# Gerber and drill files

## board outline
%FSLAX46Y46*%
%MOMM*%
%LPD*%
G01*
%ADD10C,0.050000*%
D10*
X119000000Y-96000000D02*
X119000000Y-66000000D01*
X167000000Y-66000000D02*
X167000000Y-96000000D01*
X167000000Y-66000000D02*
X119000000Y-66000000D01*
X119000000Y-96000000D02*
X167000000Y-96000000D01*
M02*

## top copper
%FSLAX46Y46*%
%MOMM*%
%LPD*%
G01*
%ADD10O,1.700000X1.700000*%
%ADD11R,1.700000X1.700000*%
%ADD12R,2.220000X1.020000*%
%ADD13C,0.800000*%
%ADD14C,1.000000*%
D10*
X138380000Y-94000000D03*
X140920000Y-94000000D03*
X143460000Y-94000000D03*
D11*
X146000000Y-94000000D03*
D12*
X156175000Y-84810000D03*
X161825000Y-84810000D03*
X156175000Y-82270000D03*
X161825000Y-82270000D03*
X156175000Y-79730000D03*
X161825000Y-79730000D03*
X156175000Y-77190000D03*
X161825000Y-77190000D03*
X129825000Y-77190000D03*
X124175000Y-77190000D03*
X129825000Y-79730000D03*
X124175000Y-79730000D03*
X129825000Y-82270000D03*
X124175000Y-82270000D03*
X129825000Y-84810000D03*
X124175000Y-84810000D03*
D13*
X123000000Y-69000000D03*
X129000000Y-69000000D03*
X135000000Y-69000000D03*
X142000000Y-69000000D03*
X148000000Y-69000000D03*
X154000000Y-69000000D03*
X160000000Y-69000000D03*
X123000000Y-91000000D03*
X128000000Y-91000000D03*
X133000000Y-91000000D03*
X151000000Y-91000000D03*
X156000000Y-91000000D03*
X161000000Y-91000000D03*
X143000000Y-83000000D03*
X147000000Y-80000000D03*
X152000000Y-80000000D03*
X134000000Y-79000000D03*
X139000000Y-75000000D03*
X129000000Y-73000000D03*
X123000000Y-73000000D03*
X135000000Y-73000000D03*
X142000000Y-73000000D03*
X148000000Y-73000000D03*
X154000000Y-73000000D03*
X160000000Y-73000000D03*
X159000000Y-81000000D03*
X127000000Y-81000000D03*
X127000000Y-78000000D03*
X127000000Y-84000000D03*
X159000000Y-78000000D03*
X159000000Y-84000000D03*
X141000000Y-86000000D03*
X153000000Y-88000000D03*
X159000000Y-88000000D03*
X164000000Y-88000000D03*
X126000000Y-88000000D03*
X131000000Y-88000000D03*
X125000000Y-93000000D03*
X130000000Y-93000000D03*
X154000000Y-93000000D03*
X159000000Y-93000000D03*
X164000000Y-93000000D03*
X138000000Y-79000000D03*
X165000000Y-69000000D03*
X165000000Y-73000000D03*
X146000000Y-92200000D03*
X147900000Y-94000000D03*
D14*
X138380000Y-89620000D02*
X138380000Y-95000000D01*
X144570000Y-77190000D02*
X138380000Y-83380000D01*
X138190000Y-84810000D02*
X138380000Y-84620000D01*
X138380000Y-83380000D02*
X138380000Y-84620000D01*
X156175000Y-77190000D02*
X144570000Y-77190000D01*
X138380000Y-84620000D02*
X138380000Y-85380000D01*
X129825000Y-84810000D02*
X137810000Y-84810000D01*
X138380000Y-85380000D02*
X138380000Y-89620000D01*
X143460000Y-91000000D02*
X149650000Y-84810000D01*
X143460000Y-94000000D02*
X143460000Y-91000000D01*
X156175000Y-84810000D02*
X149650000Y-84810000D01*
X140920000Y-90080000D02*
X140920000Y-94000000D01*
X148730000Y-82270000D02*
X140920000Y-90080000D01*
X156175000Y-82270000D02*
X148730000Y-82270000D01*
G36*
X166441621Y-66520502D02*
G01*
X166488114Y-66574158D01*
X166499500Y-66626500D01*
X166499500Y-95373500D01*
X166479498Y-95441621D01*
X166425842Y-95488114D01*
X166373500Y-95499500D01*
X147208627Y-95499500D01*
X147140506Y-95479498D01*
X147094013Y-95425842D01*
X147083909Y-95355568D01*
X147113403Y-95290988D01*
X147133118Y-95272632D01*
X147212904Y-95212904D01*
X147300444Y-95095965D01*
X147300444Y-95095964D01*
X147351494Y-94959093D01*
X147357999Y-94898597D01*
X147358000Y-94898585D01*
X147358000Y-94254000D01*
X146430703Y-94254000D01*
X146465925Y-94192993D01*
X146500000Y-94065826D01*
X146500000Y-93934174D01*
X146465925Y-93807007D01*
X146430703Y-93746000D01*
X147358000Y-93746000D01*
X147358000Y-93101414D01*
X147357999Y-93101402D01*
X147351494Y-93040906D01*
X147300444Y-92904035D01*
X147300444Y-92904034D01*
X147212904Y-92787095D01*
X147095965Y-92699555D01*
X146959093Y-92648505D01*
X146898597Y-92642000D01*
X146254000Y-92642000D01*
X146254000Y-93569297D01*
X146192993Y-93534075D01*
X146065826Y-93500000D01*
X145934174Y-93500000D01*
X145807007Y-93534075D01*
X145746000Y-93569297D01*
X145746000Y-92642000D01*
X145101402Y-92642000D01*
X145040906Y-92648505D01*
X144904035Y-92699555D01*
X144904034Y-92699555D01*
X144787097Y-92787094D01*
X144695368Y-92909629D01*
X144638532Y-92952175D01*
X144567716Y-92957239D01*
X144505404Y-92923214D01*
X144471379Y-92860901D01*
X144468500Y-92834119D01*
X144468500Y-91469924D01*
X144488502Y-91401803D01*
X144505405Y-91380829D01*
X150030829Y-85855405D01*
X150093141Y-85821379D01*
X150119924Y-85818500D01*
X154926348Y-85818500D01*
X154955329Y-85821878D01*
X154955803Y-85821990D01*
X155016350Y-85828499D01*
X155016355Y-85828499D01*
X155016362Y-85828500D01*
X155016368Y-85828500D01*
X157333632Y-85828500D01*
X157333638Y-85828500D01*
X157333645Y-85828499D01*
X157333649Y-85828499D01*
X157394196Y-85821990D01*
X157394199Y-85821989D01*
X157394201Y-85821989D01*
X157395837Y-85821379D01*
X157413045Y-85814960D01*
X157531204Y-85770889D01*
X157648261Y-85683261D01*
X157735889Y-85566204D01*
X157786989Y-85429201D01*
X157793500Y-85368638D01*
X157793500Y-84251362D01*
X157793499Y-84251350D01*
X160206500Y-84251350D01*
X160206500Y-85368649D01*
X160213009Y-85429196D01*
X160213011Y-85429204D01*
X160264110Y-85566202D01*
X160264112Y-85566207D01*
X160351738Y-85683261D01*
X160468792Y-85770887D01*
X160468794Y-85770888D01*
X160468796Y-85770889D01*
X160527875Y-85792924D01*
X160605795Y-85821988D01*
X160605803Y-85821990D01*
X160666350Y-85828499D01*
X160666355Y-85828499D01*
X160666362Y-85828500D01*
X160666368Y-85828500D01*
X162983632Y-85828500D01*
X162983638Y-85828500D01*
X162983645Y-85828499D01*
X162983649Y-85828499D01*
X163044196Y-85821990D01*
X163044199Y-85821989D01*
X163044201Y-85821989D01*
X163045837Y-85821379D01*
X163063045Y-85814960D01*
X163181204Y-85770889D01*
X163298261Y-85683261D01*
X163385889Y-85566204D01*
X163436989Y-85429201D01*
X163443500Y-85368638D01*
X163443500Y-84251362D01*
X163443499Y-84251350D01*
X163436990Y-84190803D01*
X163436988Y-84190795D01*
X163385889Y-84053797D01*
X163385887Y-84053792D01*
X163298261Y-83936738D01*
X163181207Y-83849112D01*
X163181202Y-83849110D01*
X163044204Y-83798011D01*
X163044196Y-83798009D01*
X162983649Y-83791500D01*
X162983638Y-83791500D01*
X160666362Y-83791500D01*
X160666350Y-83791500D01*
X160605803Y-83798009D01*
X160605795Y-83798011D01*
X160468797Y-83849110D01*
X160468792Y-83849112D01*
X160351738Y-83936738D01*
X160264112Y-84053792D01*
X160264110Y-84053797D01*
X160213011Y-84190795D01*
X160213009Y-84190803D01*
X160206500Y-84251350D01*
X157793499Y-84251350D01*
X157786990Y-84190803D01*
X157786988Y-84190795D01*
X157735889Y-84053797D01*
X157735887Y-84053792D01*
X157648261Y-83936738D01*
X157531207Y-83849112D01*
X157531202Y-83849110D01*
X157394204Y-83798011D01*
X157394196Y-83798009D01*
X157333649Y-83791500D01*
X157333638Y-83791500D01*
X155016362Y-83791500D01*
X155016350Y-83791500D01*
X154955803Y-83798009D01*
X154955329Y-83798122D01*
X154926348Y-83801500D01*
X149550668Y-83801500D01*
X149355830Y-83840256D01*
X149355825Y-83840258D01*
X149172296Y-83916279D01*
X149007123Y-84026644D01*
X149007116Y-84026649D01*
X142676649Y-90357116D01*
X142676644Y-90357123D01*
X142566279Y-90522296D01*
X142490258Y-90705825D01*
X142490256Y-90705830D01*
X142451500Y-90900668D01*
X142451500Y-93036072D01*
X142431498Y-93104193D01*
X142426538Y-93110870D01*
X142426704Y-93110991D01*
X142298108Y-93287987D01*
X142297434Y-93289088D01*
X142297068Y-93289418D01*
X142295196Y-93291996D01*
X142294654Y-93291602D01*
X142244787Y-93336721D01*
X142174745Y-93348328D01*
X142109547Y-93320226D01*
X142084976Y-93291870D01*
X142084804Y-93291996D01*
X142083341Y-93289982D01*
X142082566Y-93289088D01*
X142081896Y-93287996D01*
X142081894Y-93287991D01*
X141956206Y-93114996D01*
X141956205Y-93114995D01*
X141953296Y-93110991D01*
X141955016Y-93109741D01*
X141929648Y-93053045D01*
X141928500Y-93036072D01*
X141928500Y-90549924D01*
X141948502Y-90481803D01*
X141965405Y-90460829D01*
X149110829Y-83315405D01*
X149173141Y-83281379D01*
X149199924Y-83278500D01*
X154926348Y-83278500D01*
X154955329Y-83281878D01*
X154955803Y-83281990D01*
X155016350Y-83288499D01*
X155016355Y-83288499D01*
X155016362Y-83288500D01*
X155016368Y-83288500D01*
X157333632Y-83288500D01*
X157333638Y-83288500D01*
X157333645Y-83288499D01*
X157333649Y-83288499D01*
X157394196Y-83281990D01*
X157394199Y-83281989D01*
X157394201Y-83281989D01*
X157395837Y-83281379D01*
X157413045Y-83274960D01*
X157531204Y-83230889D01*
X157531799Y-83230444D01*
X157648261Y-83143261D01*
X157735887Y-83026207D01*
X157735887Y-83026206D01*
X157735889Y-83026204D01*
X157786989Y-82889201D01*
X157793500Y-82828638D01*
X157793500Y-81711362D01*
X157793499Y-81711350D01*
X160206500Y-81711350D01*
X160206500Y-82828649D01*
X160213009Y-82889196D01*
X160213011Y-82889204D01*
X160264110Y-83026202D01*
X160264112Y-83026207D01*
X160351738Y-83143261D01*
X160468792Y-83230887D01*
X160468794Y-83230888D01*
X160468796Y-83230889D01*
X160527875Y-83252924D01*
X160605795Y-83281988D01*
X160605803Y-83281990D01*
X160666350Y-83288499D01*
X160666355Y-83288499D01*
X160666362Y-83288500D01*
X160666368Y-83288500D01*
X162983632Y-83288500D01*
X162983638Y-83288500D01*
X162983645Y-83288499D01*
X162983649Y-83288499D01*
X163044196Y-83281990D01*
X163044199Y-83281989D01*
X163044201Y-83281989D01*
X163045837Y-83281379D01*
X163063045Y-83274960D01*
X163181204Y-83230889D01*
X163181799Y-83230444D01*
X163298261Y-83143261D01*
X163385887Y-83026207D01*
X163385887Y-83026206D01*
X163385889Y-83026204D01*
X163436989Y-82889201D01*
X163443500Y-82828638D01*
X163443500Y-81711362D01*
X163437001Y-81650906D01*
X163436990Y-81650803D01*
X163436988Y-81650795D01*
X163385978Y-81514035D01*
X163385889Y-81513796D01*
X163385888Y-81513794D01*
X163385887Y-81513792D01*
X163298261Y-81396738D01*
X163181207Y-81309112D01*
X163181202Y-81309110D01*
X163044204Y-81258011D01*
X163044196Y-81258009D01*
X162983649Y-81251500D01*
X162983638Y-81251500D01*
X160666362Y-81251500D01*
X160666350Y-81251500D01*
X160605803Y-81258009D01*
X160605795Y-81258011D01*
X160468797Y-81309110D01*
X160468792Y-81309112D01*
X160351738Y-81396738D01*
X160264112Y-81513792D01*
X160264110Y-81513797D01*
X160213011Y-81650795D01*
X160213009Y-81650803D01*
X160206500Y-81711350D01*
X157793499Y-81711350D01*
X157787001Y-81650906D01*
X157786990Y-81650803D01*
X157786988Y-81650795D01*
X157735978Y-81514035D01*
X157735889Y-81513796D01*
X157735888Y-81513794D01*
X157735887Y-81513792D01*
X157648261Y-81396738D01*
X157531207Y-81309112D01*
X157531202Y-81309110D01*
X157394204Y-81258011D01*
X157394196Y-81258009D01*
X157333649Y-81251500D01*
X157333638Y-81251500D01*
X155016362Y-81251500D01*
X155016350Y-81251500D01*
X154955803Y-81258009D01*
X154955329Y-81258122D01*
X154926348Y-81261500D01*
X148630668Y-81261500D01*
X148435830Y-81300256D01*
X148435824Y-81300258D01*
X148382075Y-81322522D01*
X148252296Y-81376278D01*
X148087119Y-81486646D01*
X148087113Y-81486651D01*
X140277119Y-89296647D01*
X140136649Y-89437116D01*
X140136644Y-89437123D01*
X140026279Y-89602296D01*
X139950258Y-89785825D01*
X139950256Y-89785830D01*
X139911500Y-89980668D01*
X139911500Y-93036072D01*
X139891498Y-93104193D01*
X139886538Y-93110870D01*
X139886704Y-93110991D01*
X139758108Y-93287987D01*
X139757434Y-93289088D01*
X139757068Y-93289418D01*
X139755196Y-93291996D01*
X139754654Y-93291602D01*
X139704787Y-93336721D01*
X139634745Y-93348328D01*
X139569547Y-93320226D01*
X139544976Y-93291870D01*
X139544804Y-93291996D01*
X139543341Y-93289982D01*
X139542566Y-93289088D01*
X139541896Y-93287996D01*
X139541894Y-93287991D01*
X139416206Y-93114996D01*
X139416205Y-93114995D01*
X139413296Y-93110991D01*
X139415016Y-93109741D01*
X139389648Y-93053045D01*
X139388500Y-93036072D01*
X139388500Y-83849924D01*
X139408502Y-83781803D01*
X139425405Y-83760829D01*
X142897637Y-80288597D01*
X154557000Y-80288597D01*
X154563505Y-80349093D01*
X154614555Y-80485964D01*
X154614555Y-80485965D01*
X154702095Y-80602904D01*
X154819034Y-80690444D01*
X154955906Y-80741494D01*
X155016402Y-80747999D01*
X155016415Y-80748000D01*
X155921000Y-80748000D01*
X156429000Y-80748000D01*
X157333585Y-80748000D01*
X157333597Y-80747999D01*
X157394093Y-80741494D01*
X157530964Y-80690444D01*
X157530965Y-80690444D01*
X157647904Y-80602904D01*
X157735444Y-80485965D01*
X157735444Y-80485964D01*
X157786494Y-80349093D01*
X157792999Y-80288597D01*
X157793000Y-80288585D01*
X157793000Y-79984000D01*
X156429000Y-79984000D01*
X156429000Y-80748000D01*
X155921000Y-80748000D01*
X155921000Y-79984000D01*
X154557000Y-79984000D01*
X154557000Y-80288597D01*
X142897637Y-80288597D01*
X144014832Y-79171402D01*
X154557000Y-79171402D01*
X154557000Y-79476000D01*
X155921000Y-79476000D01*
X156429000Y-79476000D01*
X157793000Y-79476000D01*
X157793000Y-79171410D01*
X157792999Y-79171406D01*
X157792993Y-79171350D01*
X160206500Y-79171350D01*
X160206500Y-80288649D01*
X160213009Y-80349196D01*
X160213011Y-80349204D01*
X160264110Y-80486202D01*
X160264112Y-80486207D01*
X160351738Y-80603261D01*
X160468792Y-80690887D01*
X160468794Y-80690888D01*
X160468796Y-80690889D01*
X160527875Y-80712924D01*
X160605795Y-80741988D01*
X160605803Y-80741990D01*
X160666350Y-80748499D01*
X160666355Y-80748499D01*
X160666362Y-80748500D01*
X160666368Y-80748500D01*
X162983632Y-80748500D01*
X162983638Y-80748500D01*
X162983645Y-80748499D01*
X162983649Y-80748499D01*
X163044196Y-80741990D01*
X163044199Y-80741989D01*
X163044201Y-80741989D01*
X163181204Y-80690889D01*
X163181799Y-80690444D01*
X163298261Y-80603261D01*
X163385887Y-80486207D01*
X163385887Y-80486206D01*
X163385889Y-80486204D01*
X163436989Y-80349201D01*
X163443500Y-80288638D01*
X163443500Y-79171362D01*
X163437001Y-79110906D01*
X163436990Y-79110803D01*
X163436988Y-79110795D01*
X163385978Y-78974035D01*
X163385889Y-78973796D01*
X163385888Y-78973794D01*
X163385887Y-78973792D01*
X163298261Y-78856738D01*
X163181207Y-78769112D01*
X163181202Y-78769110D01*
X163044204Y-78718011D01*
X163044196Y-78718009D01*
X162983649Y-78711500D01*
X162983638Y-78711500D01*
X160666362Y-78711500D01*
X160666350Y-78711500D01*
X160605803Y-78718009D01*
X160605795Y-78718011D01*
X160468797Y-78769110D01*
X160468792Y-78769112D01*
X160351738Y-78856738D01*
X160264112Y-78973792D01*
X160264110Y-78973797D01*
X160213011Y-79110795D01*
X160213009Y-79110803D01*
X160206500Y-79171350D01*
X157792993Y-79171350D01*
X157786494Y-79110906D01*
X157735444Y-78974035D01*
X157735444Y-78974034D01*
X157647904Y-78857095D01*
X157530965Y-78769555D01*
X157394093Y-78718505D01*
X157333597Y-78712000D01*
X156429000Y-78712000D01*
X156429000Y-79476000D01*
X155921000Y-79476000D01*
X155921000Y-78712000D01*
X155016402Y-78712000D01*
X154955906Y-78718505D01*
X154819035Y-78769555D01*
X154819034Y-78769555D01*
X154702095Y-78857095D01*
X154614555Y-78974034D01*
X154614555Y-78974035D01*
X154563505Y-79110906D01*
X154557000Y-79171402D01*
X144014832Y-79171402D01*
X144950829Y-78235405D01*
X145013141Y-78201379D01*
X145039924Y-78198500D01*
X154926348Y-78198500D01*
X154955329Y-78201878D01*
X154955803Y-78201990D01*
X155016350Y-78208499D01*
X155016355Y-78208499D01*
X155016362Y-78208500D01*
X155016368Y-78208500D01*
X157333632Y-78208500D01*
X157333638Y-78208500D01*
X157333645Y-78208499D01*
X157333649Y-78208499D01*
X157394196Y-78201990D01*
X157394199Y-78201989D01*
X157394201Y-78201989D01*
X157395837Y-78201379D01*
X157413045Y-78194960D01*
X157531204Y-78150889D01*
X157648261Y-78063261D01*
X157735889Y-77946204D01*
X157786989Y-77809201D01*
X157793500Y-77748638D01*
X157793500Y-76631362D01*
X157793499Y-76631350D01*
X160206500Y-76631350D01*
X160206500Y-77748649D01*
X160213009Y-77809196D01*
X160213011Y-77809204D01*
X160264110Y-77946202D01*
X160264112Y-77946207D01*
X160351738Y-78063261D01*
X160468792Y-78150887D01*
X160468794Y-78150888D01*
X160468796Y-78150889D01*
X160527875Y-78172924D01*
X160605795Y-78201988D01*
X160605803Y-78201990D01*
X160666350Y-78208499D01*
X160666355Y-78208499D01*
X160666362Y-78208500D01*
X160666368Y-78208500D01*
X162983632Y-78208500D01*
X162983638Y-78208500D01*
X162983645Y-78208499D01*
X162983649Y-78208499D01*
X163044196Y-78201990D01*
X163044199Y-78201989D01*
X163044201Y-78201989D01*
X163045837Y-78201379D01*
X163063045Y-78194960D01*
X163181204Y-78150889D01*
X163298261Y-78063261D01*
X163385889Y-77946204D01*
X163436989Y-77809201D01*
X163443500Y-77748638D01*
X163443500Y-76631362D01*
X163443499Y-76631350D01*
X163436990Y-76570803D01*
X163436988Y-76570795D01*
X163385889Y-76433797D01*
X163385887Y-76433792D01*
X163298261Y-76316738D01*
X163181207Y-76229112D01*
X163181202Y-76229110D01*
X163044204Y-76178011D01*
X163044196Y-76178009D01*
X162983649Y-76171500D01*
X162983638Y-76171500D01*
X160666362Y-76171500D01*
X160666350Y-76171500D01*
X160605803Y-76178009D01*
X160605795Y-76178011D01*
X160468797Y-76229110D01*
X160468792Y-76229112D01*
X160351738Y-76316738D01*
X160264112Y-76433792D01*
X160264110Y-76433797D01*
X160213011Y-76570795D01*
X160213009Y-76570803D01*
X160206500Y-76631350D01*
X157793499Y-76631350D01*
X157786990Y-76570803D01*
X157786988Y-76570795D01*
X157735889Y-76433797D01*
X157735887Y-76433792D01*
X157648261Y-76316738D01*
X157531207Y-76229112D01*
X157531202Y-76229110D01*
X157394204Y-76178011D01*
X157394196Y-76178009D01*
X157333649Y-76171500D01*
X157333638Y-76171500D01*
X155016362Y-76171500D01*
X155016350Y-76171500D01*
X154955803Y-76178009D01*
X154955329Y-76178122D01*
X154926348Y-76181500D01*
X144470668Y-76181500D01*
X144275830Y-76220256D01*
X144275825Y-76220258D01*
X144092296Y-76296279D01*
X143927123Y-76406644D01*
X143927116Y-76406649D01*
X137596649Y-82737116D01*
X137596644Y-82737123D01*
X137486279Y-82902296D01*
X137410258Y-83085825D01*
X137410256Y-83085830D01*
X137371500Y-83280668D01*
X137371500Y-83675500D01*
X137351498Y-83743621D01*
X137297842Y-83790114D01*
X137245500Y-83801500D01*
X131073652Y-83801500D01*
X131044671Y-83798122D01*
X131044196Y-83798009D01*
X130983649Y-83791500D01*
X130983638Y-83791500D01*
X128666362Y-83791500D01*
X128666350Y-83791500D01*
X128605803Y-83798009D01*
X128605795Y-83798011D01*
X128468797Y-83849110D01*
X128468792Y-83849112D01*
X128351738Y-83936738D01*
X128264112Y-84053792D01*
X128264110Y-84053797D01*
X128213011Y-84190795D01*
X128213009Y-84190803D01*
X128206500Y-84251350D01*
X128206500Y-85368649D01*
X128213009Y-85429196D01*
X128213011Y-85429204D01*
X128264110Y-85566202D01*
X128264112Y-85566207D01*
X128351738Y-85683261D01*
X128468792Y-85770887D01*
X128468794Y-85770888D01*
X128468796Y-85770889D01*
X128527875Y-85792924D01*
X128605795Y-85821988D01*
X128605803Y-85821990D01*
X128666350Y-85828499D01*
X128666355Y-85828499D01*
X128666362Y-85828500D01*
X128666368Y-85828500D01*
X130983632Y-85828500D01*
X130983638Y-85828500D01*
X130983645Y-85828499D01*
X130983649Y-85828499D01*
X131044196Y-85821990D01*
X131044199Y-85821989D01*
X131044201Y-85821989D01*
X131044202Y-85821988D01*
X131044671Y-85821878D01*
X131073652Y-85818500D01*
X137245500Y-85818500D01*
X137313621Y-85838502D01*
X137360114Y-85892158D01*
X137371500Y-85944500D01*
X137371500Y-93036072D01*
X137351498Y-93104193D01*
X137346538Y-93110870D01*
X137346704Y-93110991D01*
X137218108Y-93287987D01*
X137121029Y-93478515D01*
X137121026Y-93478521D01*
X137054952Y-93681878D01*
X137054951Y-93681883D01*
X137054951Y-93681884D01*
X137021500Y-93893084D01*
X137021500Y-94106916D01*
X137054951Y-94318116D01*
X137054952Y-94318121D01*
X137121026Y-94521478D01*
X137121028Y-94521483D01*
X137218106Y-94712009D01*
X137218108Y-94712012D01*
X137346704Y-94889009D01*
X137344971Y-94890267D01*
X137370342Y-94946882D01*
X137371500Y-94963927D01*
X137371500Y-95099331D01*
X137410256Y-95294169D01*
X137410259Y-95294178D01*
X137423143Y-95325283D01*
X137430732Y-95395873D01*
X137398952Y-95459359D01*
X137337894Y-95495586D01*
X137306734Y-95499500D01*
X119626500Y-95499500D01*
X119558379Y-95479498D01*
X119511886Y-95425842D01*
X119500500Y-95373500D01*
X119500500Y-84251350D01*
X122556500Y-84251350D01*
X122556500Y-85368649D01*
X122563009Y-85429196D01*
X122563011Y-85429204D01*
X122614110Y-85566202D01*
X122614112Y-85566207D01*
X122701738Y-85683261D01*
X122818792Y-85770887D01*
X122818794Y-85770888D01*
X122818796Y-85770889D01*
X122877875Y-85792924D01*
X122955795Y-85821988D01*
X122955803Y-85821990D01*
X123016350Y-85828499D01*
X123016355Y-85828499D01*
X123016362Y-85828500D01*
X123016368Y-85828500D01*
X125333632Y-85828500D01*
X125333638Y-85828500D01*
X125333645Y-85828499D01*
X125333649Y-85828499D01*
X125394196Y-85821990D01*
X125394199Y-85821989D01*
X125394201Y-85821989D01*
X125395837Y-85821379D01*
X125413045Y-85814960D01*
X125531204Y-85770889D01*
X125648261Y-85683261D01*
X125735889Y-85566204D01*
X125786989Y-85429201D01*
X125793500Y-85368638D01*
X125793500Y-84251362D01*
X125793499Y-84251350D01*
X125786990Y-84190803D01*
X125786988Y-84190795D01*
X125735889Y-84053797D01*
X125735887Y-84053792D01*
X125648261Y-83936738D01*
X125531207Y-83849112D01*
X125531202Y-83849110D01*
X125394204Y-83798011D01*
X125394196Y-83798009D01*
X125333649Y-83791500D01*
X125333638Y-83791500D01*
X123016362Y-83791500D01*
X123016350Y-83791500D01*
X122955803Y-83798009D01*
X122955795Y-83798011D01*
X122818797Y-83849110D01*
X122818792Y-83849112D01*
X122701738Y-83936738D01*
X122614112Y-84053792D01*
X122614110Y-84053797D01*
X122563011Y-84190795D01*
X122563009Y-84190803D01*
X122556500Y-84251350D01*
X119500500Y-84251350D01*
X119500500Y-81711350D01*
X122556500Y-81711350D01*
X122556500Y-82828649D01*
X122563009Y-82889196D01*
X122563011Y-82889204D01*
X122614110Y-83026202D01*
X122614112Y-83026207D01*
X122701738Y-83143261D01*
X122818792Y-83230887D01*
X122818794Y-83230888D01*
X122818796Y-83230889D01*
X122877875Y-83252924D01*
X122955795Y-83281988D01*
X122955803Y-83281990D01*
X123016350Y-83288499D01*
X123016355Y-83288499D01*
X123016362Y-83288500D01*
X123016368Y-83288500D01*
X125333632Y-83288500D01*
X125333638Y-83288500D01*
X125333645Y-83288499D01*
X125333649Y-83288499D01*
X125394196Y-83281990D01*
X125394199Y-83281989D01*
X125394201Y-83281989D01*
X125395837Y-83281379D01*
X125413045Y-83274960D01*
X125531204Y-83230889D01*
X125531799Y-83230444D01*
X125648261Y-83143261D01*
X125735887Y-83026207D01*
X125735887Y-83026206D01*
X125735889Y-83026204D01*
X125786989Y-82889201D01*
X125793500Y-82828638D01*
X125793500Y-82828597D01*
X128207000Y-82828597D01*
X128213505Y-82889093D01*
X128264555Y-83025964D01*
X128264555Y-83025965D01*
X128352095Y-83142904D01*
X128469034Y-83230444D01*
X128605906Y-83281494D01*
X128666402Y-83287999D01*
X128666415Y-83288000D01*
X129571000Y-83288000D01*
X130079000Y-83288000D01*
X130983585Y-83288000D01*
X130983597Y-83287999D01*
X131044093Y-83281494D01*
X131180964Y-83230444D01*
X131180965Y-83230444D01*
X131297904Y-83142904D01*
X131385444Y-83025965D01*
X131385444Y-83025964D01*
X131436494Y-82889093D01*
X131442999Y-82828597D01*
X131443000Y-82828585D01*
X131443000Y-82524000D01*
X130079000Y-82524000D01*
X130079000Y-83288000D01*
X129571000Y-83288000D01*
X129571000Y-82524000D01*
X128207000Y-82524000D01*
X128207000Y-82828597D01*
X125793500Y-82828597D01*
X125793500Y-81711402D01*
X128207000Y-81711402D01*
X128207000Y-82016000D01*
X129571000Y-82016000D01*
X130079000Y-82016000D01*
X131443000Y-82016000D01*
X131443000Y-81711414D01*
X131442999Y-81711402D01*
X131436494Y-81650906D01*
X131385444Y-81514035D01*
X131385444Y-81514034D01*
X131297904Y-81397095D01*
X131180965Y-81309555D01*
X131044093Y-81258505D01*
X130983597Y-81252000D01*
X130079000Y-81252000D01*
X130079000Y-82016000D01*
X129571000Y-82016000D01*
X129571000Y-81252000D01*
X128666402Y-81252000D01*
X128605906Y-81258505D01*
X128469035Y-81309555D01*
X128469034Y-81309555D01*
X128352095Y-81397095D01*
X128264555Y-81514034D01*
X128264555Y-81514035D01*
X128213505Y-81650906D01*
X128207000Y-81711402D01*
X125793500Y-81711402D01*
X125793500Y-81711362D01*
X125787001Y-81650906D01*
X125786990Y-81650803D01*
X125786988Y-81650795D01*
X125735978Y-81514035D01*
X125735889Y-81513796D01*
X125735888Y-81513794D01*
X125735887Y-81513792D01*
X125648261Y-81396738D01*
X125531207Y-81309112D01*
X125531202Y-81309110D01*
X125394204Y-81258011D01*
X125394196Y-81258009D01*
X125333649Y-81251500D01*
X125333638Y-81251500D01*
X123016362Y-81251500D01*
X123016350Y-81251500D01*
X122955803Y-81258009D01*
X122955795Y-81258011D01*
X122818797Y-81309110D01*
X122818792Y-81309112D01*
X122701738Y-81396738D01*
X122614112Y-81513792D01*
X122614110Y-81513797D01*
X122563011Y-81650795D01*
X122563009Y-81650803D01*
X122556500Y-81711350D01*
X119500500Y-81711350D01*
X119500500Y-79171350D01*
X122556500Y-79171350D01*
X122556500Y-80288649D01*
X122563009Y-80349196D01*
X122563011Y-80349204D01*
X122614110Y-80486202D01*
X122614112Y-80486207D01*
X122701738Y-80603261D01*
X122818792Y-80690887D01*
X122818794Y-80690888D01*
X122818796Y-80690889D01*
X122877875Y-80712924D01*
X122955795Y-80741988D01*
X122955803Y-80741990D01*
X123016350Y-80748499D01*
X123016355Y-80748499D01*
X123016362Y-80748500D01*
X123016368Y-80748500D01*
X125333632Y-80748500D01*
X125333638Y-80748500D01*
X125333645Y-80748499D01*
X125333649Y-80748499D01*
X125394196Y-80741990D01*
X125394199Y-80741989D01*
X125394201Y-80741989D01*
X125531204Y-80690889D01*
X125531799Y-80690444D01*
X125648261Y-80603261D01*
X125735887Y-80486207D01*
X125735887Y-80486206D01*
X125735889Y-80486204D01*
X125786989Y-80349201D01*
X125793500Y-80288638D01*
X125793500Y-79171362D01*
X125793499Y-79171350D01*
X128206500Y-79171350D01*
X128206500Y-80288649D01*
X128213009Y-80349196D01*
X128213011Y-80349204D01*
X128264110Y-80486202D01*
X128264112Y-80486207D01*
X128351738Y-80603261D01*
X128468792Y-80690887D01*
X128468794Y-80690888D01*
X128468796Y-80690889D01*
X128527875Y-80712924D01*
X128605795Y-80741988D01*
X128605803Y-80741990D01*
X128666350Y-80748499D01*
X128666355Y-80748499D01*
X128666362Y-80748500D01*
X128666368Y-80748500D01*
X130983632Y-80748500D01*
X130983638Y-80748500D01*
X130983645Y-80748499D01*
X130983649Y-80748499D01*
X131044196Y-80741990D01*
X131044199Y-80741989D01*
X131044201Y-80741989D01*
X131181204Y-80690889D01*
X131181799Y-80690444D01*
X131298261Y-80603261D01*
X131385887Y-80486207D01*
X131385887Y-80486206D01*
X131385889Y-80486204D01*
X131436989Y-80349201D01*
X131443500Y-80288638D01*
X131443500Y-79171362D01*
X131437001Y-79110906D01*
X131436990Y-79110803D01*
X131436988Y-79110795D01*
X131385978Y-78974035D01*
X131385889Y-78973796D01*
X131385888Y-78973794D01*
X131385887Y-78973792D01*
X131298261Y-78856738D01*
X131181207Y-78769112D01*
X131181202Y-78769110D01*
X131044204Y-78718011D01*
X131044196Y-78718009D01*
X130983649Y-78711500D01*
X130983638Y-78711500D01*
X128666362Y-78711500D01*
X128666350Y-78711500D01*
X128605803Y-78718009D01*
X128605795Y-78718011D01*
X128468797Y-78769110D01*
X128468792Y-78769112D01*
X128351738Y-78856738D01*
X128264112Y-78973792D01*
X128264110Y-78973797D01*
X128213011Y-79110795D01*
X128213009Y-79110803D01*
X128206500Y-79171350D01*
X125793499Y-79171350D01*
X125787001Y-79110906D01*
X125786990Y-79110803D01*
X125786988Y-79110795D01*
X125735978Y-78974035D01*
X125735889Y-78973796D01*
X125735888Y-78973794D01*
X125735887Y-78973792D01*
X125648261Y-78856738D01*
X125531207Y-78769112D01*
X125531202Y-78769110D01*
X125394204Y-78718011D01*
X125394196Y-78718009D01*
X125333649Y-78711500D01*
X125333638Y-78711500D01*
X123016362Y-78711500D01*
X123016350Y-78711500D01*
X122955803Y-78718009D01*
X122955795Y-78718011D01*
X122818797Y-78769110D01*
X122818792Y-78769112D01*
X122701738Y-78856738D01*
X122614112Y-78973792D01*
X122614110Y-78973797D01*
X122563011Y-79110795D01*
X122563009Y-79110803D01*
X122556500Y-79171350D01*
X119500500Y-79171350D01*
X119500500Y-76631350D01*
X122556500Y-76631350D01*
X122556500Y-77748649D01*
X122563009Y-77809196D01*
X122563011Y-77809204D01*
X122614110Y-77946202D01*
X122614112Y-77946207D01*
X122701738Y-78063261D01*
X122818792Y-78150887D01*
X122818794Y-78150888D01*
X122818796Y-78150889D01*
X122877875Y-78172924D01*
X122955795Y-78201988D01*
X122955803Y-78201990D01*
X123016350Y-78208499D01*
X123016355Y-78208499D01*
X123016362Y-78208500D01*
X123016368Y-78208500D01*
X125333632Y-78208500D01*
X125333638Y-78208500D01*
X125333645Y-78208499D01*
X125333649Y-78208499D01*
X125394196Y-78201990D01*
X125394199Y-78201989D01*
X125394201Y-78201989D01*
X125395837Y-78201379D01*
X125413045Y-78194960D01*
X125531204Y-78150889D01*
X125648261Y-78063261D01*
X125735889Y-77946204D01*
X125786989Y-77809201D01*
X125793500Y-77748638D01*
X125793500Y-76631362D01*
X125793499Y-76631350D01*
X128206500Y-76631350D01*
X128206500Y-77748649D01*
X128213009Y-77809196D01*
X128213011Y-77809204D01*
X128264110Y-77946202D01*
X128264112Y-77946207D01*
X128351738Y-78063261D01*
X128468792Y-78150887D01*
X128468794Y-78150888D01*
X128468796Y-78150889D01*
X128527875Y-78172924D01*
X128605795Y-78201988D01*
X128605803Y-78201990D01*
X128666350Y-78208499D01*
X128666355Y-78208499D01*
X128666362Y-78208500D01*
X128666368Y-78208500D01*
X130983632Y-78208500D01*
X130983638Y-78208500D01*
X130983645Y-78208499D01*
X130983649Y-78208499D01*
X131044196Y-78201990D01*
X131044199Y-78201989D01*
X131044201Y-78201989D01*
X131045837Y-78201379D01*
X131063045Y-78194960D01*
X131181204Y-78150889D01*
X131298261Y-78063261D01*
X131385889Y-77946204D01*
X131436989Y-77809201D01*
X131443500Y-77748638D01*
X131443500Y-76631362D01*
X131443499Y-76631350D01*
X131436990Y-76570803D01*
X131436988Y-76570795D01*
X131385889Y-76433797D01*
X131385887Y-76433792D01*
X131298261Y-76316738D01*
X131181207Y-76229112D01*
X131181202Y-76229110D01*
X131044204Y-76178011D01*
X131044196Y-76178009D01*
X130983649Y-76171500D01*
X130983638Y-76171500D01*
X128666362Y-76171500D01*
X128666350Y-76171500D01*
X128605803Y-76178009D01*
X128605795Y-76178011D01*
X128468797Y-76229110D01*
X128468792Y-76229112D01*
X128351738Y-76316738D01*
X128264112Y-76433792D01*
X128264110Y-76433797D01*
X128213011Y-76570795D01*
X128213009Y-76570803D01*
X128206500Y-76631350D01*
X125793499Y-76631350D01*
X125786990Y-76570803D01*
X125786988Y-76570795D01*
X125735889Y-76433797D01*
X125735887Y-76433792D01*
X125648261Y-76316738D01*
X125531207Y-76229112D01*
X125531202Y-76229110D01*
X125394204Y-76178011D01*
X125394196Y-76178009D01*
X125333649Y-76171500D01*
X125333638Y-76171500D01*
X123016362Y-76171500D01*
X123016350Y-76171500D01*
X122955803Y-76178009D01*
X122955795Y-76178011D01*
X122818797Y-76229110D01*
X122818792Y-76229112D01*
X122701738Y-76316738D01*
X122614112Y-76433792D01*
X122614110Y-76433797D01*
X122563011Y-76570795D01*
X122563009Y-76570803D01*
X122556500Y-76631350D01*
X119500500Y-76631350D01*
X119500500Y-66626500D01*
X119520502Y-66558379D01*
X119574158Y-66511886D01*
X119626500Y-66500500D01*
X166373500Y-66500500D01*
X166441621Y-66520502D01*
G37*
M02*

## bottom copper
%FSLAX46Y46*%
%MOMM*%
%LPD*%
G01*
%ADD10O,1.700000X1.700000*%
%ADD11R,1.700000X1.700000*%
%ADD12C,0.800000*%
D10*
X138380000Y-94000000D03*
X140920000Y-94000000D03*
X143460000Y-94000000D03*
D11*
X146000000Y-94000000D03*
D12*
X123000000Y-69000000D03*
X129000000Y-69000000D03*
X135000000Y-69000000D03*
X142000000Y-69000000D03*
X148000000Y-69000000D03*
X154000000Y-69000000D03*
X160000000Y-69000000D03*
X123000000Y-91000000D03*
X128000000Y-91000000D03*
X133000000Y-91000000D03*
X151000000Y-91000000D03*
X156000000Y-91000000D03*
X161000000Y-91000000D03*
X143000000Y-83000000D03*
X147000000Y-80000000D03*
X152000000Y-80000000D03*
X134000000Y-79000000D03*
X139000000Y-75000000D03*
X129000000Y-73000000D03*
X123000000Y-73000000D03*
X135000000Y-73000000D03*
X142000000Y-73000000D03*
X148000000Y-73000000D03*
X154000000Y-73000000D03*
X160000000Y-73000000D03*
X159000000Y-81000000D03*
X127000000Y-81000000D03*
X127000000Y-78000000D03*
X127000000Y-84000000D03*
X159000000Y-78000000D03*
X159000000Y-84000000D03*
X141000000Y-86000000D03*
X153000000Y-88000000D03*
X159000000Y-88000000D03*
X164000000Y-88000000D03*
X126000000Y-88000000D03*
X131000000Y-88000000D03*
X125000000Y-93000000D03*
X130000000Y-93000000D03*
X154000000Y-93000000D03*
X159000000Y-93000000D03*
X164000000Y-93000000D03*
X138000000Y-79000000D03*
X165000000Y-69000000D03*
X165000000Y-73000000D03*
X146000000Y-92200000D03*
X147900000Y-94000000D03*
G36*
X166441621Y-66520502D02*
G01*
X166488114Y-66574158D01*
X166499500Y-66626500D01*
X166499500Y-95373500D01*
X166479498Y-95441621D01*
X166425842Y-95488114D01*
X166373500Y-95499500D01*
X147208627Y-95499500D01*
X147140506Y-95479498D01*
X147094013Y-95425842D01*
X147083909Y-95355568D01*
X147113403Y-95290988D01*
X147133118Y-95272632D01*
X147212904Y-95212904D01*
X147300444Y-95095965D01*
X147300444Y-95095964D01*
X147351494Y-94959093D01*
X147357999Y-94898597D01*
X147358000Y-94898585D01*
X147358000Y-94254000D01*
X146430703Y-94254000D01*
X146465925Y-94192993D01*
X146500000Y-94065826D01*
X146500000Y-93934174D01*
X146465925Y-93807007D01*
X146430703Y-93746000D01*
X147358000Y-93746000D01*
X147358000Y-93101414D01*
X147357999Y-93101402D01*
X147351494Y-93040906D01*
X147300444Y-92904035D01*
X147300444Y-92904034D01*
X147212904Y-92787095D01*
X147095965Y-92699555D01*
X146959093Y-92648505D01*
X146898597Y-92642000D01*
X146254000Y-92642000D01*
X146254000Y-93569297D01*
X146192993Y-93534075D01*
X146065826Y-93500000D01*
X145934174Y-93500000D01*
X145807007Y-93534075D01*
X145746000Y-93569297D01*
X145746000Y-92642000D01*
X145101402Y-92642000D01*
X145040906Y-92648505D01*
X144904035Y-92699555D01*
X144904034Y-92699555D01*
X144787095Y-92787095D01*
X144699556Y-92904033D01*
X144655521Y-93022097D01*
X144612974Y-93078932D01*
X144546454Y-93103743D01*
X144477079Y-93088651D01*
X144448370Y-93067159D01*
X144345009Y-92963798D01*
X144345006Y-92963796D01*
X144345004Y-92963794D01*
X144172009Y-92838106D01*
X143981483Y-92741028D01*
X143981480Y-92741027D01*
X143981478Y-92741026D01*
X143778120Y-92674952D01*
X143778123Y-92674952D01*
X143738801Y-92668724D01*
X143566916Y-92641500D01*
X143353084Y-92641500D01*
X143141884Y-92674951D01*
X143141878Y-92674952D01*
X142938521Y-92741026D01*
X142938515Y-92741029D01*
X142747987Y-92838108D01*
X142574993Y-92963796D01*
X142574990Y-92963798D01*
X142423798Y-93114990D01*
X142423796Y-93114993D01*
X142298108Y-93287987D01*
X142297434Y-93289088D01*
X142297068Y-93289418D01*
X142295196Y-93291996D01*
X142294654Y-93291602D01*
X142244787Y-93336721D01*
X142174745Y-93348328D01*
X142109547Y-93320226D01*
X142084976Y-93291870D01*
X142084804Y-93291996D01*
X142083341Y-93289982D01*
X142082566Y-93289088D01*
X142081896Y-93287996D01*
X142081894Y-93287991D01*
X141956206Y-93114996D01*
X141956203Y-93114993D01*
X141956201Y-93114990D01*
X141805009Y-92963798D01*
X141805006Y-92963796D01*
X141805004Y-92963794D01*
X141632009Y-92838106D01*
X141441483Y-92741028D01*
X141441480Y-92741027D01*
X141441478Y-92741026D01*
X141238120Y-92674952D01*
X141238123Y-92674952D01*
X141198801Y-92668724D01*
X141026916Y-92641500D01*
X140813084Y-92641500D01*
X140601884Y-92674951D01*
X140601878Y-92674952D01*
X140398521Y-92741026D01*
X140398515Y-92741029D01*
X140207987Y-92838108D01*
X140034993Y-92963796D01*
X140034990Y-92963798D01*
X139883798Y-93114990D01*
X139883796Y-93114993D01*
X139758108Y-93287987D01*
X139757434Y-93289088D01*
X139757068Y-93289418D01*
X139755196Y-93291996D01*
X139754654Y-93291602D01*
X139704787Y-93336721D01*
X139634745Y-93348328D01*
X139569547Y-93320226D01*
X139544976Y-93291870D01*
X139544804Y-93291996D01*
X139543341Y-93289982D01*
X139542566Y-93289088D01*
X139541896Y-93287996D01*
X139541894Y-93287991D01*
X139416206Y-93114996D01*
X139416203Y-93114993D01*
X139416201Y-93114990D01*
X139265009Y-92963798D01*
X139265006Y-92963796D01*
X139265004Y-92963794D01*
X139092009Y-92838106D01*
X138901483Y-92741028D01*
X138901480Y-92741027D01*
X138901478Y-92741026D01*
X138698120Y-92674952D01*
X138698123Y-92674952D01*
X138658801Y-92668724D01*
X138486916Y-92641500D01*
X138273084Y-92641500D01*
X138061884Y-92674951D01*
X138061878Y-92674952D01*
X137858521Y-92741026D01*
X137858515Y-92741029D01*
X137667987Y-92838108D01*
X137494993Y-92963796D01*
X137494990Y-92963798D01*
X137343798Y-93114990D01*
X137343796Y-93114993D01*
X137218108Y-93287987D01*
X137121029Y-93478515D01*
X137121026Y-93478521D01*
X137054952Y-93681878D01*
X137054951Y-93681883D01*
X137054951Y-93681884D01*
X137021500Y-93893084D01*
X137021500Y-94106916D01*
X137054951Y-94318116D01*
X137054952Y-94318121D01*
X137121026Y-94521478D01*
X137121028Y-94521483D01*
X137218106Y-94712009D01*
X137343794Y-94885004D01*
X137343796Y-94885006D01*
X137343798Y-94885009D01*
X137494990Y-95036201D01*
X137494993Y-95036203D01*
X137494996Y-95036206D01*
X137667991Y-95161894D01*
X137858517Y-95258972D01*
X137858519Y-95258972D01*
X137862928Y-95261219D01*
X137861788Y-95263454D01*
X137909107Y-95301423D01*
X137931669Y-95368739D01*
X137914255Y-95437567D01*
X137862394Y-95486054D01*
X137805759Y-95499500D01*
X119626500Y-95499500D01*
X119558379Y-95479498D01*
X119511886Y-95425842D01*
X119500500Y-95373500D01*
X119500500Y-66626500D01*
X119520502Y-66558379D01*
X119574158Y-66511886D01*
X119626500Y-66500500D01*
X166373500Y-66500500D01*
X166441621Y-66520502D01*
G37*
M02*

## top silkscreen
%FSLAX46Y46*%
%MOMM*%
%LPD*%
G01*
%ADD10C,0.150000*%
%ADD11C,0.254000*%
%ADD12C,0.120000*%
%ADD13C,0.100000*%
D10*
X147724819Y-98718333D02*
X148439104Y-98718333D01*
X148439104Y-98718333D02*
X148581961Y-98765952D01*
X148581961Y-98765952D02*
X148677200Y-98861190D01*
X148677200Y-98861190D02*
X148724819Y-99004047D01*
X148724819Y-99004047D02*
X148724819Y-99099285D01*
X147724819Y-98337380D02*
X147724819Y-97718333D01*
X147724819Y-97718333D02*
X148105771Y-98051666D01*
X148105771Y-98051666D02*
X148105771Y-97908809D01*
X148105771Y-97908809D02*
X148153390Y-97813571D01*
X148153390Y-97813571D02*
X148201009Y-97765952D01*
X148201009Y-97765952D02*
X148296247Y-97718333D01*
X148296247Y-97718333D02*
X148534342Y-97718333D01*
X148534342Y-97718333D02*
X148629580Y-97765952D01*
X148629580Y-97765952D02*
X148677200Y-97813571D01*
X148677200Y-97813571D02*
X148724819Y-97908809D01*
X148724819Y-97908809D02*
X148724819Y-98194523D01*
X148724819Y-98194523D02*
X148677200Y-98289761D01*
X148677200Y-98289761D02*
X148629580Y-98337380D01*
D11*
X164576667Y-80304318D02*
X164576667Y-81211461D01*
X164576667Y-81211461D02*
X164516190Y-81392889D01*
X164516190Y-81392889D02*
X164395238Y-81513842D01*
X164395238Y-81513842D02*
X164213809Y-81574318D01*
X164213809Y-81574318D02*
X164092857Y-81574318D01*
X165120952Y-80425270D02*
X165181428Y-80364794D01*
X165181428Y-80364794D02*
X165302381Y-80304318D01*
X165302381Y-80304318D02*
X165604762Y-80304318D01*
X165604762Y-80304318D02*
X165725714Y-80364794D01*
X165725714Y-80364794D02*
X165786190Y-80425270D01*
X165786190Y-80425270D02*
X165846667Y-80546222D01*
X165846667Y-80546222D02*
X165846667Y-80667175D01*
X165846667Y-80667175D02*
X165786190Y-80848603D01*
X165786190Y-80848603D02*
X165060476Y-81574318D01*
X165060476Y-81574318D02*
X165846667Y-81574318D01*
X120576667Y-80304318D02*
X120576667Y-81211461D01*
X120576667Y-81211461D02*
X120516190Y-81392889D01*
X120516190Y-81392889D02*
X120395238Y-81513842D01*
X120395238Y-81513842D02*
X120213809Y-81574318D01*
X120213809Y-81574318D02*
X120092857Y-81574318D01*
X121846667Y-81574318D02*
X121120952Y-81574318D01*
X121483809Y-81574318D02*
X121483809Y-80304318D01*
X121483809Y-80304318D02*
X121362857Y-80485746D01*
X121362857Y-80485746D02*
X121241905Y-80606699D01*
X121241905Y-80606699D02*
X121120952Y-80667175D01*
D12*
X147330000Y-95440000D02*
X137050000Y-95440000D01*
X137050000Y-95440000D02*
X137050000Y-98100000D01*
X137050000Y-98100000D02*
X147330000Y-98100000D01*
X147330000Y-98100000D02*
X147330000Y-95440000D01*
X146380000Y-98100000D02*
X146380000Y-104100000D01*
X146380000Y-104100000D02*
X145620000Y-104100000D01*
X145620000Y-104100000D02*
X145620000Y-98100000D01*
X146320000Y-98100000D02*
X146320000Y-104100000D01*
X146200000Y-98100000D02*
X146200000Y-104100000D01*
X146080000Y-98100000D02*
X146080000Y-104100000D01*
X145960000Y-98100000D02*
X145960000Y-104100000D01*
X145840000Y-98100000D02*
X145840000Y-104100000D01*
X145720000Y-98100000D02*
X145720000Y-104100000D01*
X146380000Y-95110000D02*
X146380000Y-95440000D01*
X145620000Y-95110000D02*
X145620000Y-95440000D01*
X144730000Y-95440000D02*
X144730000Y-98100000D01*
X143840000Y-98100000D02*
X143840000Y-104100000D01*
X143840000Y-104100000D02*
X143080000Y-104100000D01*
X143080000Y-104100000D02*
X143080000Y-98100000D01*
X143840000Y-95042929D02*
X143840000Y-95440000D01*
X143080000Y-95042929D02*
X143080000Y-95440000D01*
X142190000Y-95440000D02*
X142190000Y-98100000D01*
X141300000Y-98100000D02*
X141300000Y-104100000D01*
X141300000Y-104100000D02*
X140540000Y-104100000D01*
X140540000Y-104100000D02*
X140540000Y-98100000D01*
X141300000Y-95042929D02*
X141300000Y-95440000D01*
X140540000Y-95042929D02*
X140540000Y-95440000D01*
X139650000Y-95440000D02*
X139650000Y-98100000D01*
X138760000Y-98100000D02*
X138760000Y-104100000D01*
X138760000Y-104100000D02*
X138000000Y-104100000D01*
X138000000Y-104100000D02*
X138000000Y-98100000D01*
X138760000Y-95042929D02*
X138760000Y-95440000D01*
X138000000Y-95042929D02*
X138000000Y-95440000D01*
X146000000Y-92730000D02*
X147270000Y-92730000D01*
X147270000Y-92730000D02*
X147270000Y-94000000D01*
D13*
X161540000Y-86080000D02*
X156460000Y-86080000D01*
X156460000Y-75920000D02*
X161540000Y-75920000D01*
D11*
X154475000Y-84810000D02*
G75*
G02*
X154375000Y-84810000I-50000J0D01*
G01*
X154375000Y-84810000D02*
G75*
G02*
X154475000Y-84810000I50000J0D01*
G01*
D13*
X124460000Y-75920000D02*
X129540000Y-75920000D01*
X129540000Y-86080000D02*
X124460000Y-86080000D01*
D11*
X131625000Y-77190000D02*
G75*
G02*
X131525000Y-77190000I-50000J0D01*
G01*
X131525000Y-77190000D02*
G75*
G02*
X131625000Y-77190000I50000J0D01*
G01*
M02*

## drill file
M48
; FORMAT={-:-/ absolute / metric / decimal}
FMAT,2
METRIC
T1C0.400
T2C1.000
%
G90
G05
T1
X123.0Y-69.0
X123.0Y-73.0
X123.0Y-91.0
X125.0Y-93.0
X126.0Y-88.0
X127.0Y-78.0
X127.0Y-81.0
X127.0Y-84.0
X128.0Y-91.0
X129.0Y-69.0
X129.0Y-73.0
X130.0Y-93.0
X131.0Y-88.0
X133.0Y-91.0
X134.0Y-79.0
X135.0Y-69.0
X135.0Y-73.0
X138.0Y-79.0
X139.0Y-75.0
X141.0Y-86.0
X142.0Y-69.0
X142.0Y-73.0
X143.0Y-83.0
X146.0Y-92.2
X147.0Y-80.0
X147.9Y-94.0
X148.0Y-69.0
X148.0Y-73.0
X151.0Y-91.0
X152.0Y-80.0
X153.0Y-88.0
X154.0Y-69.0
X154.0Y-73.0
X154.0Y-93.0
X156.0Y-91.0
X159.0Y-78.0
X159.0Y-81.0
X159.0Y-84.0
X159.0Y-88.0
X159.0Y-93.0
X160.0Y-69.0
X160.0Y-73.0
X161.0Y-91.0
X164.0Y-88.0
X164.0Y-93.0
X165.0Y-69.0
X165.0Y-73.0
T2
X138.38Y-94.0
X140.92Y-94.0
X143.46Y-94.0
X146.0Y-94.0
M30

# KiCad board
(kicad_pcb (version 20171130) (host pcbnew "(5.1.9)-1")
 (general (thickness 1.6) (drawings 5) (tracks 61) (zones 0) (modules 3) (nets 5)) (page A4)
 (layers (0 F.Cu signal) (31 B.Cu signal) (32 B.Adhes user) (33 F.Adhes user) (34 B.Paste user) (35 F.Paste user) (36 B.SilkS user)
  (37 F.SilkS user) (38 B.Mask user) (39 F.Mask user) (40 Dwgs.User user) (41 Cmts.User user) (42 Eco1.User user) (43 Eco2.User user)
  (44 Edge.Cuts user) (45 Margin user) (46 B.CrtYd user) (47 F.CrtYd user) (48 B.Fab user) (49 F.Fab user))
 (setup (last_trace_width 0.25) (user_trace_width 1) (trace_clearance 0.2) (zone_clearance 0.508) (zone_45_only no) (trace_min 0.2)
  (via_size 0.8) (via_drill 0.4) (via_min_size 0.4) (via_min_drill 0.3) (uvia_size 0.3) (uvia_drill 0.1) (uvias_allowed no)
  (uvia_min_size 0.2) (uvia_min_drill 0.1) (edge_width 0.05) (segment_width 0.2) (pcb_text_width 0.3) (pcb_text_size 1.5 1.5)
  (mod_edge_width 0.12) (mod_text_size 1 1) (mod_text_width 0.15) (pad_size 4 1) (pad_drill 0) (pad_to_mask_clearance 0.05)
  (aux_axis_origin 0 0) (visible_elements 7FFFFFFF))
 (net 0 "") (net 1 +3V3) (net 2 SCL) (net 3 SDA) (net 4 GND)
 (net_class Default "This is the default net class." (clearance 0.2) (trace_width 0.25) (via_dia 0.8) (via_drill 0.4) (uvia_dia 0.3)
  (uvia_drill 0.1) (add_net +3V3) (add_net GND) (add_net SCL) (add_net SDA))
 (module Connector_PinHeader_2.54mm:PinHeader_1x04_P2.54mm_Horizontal (layer F.Cu) (at 146 94 270)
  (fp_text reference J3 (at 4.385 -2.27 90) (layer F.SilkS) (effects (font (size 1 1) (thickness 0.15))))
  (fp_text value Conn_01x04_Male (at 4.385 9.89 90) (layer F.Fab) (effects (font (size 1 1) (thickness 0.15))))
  (fp_line (start 1.44 -1.33) (end 1.44 8.95) (layer F.SilkS) (width 0.12))
  (fp_line (start 1.44 8.95) (end 4.1 8.95) (layer F.SilkS) (width 0.12))
  (fp_line (start 4.1 8.95) (end 4.1 -1.33) (layer F.SilkS) (width 0.12))
  (fp_line (start 4.1 -1.33) (end 1.44 -1.33) (layer F.SilkS) (width 0.12))
  (fp_line (start 4.1 -0.38) (end 10.1 -0.38) (layer F.SilkS) (width 0.12))
  (fp_line (start 10.1 -0.38) (end 10.1 0.38) (layer F.SilkS) (width 0.12))
  (fp_line (start 10.1 0.38) (end 4.1 0.38) (layer F.SilkS) (width 0.12))
  (fp_line (start 4.1 -0.32) (end 10.1 -0.32) (layer F.SilkS) (width 0.12))
  (fp_line (start 4.1 -0.2) (end 10.1 -0.2) (layer F.SilkS) (width 0.12))
  (fp_line (start 4.1 -0.08) (end 10.1 -0.08) (layer F.SilkS) (width 0.12))
  (fp_line (start 4.1 0.04) (end 10.1 0.04) (layer F.SilkS) (width 0.12))
  (fp_line (start 4.1 0.16) (end 10.1 0.16) (layer F.SilkS) (width 0.12))
  (fp_line (start 4.1 0.28) (end 10.1 0.28) (layer F.SilkS) (width 0.12))
  (fp_line (start 1.11 -0.38) (end 1.44 -0.38) (layer F.SilkS) (width 0.12))
  (fp_line (start 1.11 0.38) (end 1.44 0.38) (layer F.SilkS) (width 0.12))
  (fp_line (start 1.44 1.27) (end 4.1 1.27) (layer F.SilkS) (width 0.12))
  (fp_line (start 4.1 2.16) (end 10.1 2.16) (layer F.SilkS) (width 0.12))
  (fp_line (start 10.1 2.16) (end 10.1 2.92) (layer F.SilkS) (width 0.12))
  (fp_line (start 10.1 2.92) (end 4.1 2.92) (layer F.SilkS) (width 0.12))
  (fp_line (start 1.042929 2.16) (end 1.44 2.16) (layer F.SilkS) (width 0.12))
  (fp_line (start 1.042929 2.92) (end 1.44 2.92) (layer F.SilkS) (width 0.12))
  (fp_line (start 1.44 3.81) (end 4.1 3.81) (layer F.SilkS) (width 0.12))
  (fp_line (start 4.1 4.7) (end 10.1 4.7) (layer F.SilkS) (width 0.12))
  (fp_line (start 10.1 4.7) (end 10.1 5.46) (layer F.SilkS) (width 0.12))
  (fp_line (start 10.1 5.46) (end 4.1 5.46) (layer F.SilkS) (width 0.12))
  (fp_line (start 1.042929 4.7) (end 1.44 4.7) (layer F.SilkS) (width 0.12))
  (fp_line (start 1.042929 5.46) (end 1.44 5.46) (layer F.SilkS) (width 0.12))
  (fp_line (start 1.44 6.35) (end 4.1 6.35) (layer F.SilkS) (width 0.12))
  (fp_line (start 4.1 7.24) (end 10.1 7.24) (layer F.SilkS) (width 0.12))
  (fp_line (start 10.1 7.24) (end 10.1 8) (layer F.SilkS) (width 0.12))
  (fp_line (start 10.1 8) (end 4.1 8) (layer F.SilkS) (width 0.12))
  (fp_line (start 1.042929 7.24) (end 1.44 7.24) (layer F.SilkS) (width 0.12))
  (fp_line (start 1.042929 8) (end 1.44 8) (layer F.SilkS) (width 0.12))
  (fp_line (start -1.27 0) (end -1.27 -1.27) (layer F.SilkS) (width 0.12))
  (fp_line (start -1.27 -1.27) (end 0 -1.27) (layer F.SilkS) (width 0.12))
  (pad 4 thru_hole oval (at 0 7.62 270) (size 1.7 1.7) (drill 1) (layers *.Cu *.Mask) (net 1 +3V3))
  (pad 3 thru_hole oval (at 0 5.08 270) (size 1.7 1.7) (drill 1) (layers *.Cu *.Mask) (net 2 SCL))
  (pad 2 thru_hole oval (at 0 2.54 270) (size 1.7 1.7) (drill 1) (layers *.Cu *.Mask) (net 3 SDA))
  (pad 1 thru_hole rect (at 0 0 270) (size 1.7 1.7) (drill 1) (layers *.Cu *.Mask) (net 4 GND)))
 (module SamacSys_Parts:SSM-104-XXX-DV (layer F.Cu) (at 159 81 270)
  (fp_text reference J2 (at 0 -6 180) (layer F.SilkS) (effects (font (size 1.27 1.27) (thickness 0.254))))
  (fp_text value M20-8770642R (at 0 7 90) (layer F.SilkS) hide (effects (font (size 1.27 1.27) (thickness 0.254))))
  (fp_line (start 5.08 -2.54) (end 5.08 2.54) (layer F.SilkS) (width 0.1))
  (fp_line (start -5.08 2.54) (end -5.08 -2.54) (layer F.SilkS) (width 0.1))
  (fp_circle (center 3.81 4.575) (end 3.76 4.575) (layer F.SilkS) (width 0.254))
  (pad 1 smd rect (at 3.81 2.825 270) (size 1.02 2.22) (layers F.Cu F.Paste F.Mask) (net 3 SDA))
  (pad 2 smd rect (at 3.81 -2.825 270) (size 1.02 2.22) (layers F.Cu F.Paste F.Mask))
  (pad 3 smd rect (at 1.27 2.825 270) (size 1.02 2.22) (layers F.Cu F.Paste F.Mask) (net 2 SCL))
  (pad 4 smd rect (at 1.27 -2.825 270) (size 1.02 2.22) (layers F.Cu F.Paste F.Mask))
  (pad 5 smd rect (at -1.27 2.825 270) (size 1.02 2.22) (layers F.Cu F.Paste F.Mask) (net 4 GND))
  (pad 6 smd rect (at -1.27 -2.825 270) (size 1.02 2.22) (layers F.Cu F.Paste F.Mask))
  (pad 7 smd rect (at -3.81 2.825 270) (size 1.02 2.22) (layers F.Cu F.Paste F.Mask) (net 1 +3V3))
  (pad 8 smd rect (at -3.81 -2.825 270) (size 1.02 2.22) (layers F.Cu F.Paste F.Mask)))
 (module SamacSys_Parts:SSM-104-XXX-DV (layer F.Cu) (at 127 81 90)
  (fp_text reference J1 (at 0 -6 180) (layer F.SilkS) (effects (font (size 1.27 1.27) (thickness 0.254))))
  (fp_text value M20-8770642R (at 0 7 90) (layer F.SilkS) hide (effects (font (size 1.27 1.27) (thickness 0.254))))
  (fp_line (start 5.08 -2.54) (end 5.08 2.54) (layer F.SilkS) (width 0.1))
  (fp_line (start -5.08 2.54) (end -5.08 -2.54) (layer F.SilkS) (width 0.1))
  (fp_circle (center 3.81 4.575) (end 3.76 4.575) (layer F.SilkS) (width 0.254))
  (pad 1 smd rect (at 3.81 2.825 90) (size 1.02 2.22) (layers F.Cu F.Paste F.Mask))
  (pad 2 smd rect (at 3.81 -2.825 90) (size 1.02 2.22) (layers F.Cu F.Paste F.Mask))
  (pad 3 smd rect (at 1.27 2.825 90) (size 1.02 2.22) (layers F.Cu F.Paste F.Mask))
  (pad 4 smd rect (at 1.27 -2.825 90) (size 1.02 2.22) (layers F.Cu F.Paste F.Mask))
  (pad 5 smd rect (at -1.27 2.825 90) (size 1.02 2.22) (layers F.Cu F.Paste F.Mask) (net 4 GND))
  (pad 6 smd rect (at -1.27 -2.825 90) (size 1.02 2.22) (layers F.Cu F.Paste F.Mask))
  (pad 7 smd rect (at -3.81 2.825 90) (size 1.02 2.22) (layers F.Cu F.Paste F.Mask) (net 1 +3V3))
  (pad 8 smd rect (at -3.81 -2.825 90) (size 1.02 2.22) (layers F.Cu F.Paste F.Mask)))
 (gr_line (start 119 96) (end 119 66) (layer Edge.Cuts) (width 0.05))
 (gr_line (start 167 66) (end 167 96) (layer Edge.Cuts) (width 0.05))
 (gr_line (start 167 66) (end 119 66) (layer Edge.Cuts) (width 0.05))
 (gr_line (start 119 96) (end 167 96) (layer Edge.Cuts) (width 0.05))
 (via (at 123 69) (size 0.8) (drill 0.4) (layers F.Cu B.Cu) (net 4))
 (via (at 129 69) (size 0.8) (drill 0.4) (layers F.Cu B.Cu) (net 4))
 (via (at 135 69) (size 0.8) (drill 0.4) (layers F.Cu B.Cu) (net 4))
 (via (at 142 69) (size 0.8) (drill 0.4) (layers F.Cu B.Cu) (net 4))
 (via (at 148 69) (size 0.8) (drill 0.4) (layers F.Cu B.Cu) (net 4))
 (via (at 154 69) (size 0.8) (drill 0.4) (layers F.Cu B.Cu) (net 4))
 (via (at 160 69) (size 0.8) (drill 0.4) (layers F.Cu B.Cu) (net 4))
 (via (at 123 91) (size 0.8) (drill 0.4) (layers F.Cu B.Cu) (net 4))
 (via (at 128 91) (size 0.8) (drill 0.4) (layers F.Cu B.Cu) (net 4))
 (via (at 133 91) (size 0.8) (drill 0.4) (layers F.Cu B.Cu) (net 4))
 (via (at 151 91) (size 0.8) (drill 0.4) (layers F.Cu B.Cu) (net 4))
 (via (at 156 91) (size 0.8) (drill 0.4) (layers F.Cu B.Cu) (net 4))
 (via (at 161 91) (size 0.8) (drill 0.4) (layers F.Cu B.Cu) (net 4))
 (via (at 143 83) (size 0.8) (drill 0.4) (layers F.Cu B.Cu) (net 4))
 (via (at 147 80) (size 0.8) (drill 0.4) (layers F.Cu B.Cu) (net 4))
 (via (at 152 80) (size 0.8) (drill 0.4) (layers F.Cu B.Cu) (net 4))
 (via (at 134 79) (size 0.8) (drill 0.4) (layers F.Cu B.Cu) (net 4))
 (via (at 139 75) (size 0.8) (drill 0.4) (layers F.Cu B.Cu) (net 4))
 (via (at 129 73) (size 0.8) (drill 0.4) (layers F.Cu B.Cu) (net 4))
 (via (at 123 73) (size 0.8) (drill 0.4) (layers F.Cu B.Cu) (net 4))
 (via (at 135 73) (size 0.8) (drill 0.4) (layers F.Cu B.Cu) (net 4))
 (via (at 142 73) (size 0.8) (drill 0.4) (layers F.Cu B.Cu) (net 4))
 (via (at 148 73) (size 0.8) (drill 0.4) (layers F.Cu B.Cu) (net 4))
 (via (at 154 73) (size 0.8) (drill 0.4) (layers F.Cu B.Cu) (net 4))
 (via (at 160 73) (size 0.8) (drill 0.4) (layers F.Cu B.Cu) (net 4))
 (via (at 159 81) (size 0.8) (drill 0.4) (layers F.Cu B.Cu) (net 4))
 (via (at 127 81) (size 0.8) (drill 0.4) (layers F.Cu B.Cu) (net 4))
 (via (at 127 78) (size 0.8) (drill 0.4) (layers F.Cu B.Cu) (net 4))
 (via (at 127 84) (size 0.8) (drill 0.4) (layers F.Cu B.Cu) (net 4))
 (via (at 159 78) (size 0.8) (drill 0.4) (layers F.Cu B.Cu) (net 4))
 (via (at 159 84) (size 0.8) (drill 0.4) (layers F.Cu B.Cu) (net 4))
 (via (at 141 86) (size 0.8) (drill 0.4) (layers F.Cu B.Cu) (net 4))
 (via (at 153 88) (size 0.8) (drill 0.4) (layers F.Cu B.Cu) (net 4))
 (via (at 159 88) (size 0.8) (drill 0.4) (layers F.Cu B.Cu) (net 4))
 (via (at 164 88) (size 0.8) (drill 0.4) (layers F.Cu B.Cu) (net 4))
 (via (at 126 88) (size 0.8) (drill 0.4) (layers F.Cu B.Cu) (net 4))
 (via (at 131 88) (size 0.8) (drill 0.4) (layers F.Cu B.Cu) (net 4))
 (via (at 125 93) (size 0.8) (drill 0.4) (layers F.Cu B.Cu) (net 4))
 (via (at 130 93) (size 0.8) (drill 0.4) (layers F.Cu B.Cu) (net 4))
 (via (at 154 93) (size 0.8) (drill 0.4) (layers F.Cu B.Cu) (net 4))
 (via (at 159 93) (size 0.8) (drill 0.4) (layers F.Cu B.Cu) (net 4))
 (via (at 164 93) (size 0.8) (drill 0.4) (layers F.Cu B.Cu) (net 4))
 (via (at 138 79) (size 0.8) (drill 0.4) (layers F.Cu B.Cu) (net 4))
 (via (at 165 69) (size 0.8) (drill 0.4) (layers F.Cu B.Cu) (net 4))
 (via (at 165 73) (size 0.8) (drill 0.4) (layers F.Cu B.Cu) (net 4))
 (via (at 146 92.2) (size 0.8) (drill 0.4) (layers F.Cu B.Cu) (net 4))
 (via (at 147.9 94) (size 0.8) (drill 0.4) (layers F.Cu B.Cu) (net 4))
 (segment (start 138.38 89.62) (end 138.38 95) (width 1) (layer F.Cu) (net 1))
 (segment (start 144.57 77.19) (end 138.38 83.38) (width 1) (layer F.Cu) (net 1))
 (segment (start 138.19 84.81) (end 138.38 84.62) (width 1) (layer F.Cu) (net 1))
 (segment (start 138.38 83.38) (end 138.38 84.62) (width 1) (layer F.Cu) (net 1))
 (segment (start 156.175 77.19) (end 144.57 77.19) (width 1) (layer F.Cu) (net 1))
 (segment (start 138.38 84.62) (end 138.38 85.38) (width 1) (layer F.Cu) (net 1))
 (segment (start 129.825 84.81) (end 137.81 84.81) (width 1) (layer F.Cu) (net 1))
 (segment (start 138.38 85.38) (end 138.38 89.62) (width 1) (layer F.Cu) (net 1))
 (segment (start 143.46 91) (end 149.65 84.81) (width 1) (layer F.Cu) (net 3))
 (segment (start 143.46 94) (end 143.46 91) (width 1) (layer F.Cu) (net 3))
 (segment (start 156.175 84.81) (end 149.65 84.81) (width 1) (layer F.Cu) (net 3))
 (segment (start 140.92 90.08) (end 140.92 94) (width 1) (layer F.Cu) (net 2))
 (segment (start 148.73 82.27) (end 140.92 90.08) (width 1) (layer F.Cu) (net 2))
 (segment (start 156.175 82.27) (end 148.73 82.27) (width 1) (layer F.Cu) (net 2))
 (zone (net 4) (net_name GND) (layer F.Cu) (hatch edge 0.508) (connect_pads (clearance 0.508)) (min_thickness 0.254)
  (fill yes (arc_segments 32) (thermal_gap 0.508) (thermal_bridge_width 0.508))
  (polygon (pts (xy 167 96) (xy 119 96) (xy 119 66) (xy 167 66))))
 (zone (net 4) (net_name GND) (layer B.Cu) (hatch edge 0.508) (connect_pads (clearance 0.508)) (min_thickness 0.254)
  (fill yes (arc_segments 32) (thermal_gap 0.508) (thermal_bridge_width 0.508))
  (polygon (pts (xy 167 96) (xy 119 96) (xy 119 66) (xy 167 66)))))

